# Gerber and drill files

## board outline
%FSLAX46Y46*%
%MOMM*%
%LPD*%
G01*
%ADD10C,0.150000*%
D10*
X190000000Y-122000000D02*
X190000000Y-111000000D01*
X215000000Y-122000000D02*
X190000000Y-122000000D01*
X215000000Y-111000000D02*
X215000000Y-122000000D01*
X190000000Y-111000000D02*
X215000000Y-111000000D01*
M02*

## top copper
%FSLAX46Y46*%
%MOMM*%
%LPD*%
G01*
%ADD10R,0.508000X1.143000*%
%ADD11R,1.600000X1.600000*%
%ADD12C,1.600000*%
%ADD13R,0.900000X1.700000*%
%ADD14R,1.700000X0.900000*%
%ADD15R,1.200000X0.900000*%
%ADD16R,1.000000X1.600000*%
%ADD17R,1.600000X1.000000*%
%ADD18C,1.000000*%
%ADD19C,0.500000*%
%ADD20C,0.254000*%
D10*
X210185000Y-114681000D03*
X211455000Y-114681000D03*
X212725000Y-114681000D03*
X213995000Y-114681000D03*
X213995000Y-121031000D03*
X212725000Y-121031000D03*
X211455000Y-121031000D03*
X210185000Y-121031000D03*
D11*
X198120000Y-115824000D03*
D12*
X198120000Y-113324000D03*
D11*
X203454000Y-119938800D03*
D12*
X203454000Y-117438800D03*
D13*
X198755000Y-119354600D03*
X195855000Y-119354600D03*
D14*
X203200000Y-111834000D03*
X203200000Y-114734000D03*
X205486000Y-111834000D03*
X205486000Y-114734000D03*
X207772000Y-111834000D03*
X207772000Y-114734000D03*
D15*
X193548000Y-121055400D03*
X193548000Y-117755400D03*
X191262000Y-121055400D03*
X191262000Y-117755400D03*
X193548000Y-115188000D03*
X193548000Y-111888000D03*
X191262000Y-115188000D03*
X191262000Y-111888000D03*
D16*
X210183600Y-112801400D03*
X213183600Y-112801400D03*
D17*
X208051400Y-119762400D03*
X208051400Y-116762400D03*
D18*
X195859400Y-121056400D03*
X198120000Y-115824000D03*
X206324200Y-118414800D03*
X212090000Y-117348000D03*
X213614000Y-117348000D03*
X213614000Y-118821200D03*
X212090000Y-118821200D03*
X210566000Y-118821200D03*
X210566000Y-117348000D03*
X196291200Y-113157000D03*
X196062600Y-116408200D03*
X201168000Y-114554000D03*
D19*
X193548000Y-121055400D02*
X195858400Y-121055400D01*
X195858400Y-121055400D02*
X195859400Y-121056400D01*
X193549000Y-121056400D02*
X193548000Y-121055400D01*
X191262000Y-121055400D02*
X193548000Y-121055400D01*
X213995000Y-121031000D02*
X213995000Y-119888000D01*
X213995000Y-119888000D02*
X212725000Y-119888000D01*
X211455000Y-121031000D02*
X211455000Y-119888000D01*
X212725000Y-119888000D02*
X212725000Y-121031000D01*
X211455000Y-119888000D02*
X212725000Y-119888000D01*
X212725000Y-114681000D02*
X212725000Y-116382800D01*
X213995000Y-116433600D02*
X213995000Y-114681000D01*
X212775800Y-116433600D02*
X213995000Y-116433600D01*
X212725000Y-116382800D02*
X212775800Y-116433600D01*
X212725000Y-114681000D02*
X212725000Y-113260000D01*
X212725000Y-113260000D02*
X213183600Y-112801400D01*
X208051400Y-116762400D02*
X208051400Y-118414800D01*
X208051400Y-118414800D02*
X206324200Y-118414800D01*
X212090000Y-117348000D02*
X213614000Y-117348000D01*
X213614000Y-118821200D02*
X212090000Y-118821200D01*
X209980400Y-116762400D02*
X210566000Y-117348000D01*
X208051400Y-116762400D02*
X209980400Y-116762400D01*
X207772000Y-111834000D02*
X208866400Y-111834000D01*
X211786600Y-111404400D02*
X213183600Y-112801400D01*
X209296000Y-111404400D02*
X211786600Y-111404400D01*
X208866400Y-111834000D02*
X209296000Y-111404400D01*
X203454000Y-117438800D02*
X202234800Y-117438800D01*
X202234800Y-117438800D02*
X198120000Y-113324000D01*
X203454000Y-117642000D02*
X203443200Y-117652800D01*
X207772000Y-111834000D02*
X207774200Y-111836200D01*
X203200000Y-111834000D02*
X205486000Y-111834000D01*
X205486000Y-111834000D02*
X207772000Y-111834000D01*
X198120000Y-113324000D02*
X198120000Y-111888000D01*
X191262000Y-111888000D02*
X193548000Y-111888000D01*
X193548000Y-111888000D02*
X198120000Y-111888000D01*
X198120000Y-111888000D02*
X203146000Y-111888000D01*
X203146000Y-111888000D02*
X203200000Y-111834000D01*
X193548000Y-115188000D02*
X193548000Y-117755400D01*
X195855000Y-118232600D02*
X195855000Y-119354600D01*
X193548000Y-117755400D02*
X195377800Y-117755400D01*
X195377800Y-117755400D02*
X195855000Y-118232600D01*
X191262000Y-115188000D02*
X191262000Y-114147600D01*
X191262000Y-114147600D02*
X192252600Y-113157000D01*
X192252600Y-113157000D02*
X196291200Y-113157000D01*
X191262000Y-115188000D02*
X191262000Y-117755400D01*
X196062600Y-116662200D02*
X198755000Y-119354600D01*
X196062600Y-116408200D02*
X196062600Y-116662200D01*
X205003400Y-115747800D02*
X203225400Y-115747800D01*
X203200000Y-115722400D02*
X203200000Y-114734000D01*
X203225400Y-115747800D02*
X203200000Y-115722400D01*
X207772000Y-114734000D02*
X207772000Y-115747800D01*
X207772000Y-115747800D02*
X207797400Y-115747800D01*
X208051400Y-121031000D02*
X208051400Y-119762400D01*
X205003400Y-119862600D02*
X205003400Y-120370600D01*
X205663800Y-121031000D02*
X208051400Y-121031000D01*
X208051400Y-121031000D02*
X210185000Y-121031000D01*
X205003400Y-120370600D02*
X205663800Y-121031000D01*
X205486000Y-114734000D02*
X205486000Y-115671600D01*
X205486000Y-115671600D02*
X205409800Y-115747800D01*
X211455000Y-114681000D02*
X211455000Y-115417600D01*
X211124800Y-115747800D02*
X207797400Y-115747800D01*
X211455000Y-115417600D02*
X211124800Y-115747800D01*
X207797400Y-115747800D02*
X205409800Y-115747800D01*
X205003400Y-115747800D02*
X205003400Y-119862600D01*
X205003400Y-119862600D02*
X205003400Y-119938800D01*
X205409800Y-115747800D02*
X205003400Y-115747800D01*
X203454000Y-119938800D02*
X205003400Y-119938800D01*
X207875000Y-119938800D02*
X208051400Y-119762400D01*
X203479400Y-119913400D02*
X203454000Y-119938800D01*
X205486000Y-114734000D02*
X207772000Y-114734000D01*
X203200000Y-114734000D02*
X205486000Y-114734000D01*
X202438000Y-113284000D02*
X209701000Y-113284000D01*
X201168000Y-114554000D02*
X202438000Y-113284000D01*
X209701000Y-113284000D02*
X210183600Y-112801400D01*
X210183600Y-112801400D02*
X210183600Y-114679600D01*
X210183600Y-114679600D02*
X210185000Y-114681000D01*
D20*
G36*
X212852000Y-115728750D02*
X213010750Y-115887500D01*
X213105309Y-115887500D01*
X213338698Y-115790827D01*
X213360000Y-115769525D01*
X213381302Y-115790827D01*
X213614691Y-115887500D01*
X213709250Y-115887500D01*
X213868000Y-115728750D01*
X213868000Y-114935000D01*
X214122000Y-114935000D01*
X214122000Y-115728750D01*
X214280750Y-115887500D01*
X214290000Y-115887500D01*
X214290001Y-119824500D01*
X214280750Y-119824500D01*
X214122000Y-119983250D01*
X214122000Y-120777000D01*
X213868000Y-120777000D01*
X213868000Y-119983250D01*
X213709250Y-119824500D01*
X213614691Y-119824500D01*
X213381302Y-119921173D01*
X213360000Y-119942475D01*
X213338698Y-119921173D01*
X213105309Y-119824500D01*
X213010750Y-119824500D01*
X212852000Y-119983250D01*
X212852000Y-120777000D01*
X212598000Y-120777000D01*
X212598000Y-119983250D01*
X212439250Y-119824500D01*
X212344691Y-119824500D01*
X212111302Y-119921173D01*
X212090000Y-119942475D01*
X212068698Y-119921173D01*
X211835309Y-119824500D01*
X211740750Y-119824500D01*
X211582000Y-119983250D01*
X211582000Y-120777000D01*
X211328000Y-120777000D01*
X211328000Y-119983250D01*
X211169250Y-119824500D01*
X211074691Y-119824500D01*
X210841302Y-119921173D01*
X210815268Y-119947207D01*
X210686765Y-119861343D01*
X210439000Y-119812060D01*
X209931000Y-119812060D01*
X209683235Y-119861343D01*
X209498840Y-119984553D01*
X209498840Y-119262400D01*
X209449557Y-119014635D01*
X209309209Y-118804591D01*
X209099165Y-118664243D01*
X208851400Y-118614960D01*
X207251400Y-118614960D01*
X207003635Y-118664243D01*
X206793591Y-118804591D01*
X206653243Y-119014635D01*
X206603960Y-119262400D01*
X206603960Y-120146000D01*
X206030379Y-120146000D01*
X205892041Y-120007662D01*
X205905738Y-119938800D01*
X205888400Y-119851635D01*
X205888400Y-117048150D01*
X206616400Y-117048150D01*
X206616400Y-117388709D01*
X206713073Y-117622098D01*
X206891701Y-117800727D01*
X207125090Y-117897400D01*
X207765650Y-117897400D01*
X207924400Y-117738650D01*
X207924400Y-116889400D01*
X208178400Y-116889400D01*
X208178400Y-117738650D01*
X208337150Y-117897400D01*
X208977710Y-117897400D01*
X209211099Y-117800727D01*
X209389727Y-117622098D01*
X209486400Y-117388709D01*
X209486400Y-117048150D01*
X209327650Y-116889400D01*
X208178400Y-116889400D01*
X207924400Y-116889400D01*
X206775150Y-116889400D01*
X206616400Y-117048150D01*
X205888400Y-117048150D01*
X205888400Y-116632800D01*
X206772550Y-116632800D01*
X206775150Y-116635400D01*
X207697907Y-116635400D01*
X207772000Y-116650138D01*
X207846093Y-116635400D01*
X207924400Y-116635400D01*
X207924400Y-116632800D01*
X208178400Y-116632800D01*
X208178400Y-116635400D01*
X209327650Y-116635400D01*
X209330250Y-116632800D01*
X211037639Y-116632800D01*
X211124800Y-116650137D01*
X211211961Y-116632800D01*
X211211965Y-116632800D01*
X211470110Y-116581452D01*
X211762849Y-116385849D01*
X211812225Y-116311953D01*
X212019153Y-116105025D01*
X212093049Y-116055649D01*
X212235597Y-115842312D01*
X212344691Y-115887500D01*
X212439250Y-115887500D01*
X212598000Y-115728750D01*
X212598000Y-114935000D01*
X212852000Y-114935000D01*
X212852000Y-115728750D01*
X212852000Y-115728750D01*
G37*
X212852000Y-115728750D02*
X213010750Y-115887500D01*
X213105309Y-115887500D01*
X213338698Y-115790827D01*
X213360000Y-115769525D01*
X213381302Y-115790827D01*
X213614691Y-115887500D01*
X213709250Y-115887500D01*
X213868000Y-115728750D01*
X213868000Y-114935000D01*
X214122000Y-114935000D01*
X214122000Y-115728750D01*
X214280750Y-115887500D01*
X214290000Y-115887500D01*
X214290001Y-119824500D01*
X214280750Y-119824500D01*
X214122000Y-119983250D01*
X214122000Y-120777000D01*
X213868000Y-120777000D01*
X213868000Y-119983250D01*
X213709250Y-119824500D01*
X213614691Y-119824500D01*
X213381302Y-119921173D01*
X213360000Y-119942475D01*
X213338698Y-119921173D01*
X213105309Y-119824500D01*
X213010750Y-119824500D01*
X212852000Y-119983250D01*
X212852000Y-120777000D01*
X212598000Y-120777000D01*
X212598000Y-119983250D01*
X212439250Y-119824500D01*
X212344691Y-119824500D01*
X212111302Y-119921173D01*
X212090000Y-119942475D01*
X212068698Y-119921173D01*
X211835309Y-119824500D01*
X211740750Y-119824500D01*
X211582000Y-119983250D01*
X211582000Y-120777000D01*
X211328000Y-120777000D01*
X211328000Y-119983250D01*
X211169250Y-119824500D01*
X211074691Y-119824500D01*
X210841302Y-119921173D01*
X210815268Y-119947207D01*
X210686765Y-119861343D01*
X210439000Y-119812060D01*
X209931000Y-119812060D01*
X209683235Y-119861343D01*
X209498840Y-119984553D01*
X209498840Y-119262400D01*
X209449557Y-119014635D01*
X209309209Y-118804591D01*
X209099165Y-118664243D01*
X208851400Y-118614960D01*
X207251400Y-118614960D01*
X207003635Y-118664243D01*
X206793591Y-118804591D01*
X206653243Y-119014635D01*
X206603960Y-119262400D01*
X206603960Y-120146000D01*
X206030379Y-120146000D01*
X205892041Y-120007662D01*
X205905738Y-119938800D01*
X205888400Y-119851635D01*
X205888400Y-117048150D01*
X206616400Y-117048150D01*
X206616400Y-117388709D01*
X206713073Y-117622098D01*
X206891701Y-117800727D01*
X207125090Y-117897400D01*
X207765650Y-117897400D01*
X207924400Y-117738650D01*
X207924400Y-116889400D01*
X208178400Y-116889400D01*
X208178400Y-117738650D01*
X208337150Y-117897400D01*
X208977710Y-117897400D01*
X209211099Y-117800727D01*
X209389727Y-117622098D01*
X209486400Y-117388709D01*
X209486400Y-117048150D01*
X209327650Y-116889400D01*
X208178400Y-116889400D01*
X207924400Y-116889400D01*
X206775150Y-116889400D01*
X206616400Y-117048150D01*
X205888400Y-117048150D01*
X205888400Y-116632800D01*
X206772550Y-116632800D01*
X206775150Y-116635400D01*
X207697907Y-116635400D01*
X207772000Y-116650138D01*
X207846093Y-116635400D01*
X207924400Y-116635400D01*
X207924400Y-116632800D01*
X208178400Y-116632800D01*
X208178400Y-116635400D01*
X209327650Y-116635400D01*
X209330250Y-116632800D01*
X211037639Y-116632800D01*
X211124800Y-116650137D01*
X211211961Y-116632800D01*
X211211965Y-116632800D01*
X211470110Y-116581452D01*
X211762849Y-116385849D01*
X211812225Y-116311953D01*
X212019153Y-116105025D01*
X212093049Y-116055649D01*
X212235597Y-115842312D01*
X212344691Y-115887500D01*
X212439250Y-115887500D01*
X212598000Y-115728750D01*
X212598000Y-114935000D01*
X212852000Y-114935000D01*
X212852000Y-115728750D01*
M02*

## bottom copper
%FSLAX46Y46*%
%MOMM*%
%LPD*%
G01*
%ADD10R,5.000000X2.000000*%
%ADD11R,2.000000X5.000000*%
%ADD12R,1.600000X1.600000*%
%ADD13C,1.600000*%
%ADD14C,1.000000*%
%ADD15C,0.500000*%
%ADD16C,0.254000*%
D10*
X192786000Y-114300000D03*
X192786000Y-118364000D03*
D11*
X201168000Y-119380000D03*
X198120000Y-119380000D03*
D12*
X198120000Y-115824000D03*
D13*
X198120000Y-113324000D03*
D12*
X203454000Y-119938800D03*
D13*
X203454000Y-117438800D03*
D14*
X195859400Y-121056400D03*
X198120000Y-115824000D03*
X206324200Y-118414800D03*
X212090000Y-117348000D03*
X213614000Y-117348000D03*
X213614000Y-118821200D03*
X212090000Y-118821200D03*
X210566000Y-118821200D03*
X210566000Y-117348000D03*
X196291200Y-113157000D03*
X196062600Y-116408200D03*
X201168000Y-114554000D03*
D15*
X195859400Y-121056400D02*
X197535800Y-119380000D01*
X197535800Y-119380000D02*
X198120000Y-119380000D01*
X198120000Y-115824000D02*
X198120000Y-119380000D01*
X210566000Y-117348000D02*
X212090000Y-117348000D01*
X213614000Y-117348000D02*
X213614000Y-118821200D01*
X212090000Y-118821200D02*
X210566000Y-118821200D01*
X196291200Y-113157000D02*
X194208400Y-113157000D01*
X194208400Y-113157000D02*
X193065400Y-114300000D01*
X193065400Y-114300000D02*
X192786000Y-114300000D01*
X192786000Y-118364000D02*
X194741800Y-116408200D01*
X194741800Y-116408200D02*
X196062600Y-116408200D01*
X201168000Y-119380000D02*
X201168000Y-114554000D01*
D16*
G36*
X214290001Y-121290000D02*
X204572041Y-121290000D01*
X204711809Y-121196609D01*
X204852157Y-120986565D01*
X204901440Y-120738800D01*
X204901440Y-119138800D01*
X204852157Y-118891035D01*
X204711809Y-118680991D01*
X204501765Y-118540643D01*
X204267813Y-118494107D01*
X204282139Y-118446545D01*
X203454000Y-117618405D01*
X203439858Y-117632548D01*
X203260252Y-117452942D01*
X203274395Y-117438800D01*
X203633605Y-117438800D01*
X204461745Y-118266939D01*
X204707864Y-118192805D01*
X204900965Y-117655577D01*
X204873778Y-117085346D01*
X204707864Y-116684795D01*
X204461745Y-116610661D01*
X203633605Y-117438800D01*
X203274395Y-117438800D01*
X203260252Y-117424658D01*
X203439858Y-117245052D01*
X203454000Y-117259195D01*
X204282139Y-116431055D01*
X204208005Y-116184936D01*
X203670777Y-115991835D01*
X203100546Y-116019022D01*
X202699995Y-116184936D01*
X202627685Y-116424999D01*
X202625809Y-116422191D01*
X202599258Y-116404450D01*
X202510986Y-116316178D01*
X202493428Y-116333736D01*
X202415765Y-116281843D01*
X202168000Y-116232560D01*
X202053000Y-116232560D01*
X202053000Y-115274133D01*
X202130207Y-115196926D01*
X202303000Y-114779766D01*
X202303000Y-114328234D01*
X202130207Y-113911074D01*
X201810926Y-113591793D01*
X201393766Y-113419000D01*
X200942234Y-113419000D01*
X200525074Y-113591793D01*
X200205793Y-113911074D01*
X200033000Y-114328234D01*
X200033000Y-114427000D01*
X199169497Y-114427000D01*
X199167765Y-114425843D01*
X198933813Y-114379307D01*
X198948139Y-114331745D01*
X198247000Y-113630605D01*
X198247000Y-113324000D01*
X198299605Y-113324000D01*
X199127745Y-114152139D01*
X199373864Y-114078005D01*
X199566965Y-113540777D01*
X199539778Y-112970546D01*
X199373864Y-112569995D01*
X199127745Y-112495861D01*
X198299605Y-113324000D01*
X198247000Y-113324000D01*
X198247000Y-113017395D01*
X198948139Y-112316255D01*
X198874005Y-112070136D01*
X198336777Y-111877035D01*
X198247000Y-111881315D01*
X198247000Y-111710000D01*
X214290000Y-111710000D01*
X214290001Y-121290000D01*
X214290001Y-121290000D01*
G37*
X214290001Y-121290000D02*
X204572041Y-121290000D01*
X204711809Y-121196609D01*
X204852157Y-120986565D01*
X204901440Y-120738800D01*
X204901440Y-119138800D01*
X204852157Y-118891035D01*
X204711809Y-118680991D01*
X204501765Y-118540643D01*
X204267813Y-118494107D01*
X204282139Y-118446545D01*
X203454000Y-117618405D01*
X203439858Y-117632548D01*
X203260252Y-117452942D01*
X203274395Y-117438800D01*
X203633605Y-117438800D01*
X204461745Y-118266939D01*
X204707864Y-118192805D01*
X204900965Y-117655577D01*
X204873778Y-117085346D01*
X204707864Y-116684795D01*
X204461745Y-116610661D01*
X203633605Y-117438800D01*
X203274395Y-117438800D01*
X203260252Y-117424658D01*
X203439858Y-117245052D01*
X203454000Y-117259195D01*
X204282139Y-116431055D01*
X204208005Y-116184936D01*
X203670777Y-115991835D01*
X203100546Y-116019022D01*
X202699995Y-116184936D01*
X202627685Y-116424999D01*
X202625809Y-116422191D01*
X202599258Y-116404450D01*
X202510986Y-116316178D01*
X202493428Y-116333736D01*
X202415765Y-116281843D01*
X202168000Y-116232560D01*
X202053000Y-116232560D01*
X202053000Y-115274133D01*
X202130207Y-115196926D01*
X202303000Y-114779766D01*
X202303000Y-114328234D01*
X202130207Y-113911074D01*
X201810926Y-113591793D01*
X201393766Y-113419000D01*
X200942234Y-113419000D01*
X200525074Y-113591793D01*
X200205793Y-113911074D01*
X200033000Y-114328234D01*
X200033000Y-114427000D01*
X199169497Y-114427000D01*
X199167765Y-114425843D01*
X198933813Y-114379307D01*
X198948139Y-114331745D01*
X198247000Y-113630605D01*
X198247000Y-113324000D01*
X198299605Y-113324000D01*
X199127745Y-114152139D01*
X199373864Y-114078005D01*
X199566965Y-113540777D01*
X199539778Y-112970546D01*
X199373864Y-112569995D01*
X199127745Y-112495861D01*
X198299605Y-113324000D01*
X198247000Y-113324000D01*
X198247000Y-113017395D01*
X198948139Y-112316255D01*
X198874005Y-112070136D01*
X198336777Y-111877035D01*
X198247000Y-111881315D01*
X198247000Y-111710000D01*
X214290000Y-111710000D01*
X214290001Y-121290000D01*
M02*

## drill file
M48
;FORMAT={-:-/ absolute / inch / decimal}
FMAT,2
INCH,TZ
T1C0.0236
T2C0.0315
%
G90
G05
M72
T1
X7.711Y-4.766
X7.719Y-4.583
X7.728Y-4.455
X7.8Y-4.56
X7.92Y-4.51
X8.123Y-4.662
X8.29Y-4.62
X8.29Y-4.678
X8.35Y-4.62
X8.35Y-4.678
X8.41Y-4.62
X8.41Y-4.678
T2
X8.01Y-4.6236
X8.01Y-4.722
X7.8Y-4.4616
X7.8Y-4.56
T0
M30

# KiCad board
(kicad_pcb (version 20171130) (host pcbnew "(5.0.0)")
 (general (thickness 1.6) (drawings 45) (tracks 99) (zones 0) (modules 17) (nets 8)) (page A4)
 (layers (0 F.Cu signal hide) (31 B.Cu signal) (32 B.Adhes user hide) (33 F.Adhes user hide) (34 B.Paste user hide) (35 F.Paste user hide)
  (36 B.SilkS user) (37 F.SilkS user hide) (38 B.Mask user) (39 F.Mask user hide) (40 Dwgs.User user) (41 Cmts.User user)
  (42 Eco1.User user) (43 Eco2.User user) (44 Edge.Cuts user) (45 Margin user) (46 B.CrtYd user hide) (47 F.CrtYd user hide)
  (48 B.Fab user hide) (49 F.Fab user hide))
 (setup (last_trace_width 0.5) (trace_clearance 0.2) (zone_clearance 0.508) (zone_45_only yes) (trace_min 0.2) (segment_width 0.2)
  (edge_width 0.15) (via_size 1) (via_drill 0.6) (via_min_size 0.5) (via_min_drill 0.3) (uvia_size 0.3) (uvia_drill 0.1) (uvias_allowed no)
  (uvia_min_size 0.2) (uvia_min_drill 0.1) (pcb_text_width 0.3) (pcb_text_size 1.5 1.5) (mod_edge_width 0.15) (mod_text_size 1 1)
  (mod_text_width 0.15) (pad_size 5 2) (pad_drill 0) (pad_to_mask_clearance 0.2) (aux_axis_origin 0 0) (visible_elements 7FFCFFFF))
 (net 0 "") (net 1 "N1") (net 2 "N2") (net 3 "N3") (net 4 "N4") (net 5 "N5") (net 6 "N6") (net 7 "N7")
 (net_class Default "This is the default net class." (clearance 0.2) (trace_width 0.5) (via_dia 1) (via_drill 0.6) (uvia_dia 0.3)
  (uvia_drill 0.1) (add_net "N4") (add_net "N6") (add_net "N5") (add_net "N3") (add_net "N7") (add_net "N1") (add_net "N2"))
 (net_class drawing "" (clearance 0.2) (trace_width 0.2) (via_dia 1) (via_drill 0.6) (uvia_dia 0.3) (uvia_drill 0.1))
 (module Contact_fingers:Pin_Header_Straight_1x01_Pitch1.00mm (layer F.Cu) (at 192.786 114.3 180)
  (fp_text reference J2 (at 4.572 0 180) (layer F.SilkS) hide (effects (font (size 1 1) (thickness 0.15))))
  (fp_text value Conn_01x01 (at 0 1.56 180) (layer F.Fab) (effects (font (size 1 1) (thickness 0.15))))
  (pad 1 smd rect (at 0 0 180) (size 5 2) (layers B.Cu) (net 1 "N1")))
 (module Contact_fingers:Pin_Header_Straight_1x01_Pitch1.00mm (layer F.Cu) (at 192.786 118.364 180)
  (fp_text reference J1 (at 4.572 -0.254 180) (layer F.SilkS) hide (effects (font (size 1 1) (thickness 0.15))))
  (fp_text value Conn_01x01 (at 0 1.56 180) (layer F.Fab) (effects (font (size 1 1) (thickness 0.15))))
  (pad 1 smd rect (at 0 0 180) (size 5 2) (layers B.Cu) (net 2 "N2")))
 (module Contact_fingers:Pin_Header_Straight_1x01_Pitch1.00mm (layer F.Cu) (at 201.168 119.38 270)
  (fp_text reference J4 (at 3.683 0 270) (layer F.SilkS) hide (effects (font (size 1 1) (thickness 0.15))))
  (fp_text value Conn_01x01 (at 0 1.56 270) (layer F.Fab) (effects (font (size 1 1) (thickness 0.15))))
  (pad 1 smd rect (at 0 0 270) (size 5 2) (layers B.Cu) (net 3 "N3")))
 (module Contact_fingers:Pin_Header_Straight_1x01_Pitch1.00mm (layer F.Cu) (at 198.12 119.38 270)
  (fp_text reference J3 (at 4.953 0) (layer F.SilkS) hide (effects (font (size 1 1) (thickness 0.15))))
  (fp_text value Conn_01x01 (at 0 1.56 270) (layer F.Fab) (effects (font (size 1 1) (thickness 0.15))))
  (pad 1 smd rect (at 0 0 270) (size 5 2) (layers B.Cu) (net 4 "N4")))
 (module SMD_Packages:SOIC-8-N (layer F.Cu) (at 212.09 117.856)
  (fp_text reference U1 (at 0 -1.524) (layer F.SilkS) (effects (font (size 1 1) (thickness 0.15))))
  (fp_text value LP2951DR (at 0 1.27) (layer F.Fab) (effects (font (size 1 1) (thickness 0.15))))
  (pad 8 smd rect (at -1.905 -3.175) (size 0.508 1.143) (layers F.Cu F.Paste F.Mask) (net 3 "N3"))
  (pad 7 smd rect (at -0.635 -3.175) (size 0.508 1.143) (layers F.Cu F.Paste F.Mask) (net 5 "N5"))
  (pad 6 smd rect (at 0.635 -3.175) (size 0.508 1.143) (layers F.Cu F.Paste F.Mask) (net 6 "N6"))
  (pad 5 smd rect (at 1.905 -3.175) (size 0.508 1.143) (layers F.Cu F.Paste F.Mask) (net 6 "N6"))
  (pad 4 smd rect (at 1.905 3.175) (size 0.508 1.143) (layers F.Cu F.Paste F.Mask) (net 6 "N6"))
  (pad 3 smd rect (at 0.635 3.175) (size 0.508 1.143) (layers F.Cu F.Paste F.Mask) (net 6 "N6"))
  (pad 2 smd rect (at -0.635 3.175) (size 0.508 1.143) (layers F.Cu F.Paste F.Mask) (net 6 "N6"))
  (pad 1 smd rect (at -1.905 3.175) (size 0.508 1.143) (layers F.Cu F.Paste F.Mask) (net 5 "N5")))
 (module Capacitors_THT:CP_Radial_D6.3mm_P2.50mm (layer F.Cu) (at 198.12 115.824 90)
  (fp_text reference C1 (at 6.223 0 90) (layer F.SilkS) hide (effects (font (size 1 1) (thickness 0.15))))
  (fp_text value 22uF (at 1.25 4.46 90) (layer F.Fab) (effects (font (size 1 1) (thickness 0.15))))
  (pad 1 thru_hole rect (at 0 0 90) (size 1.6 1.6) (drill 0.8) (layers *.Cu *.Mask) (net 4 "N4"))
  (pad 2 thru_hole circle (at 2.5 0 90) (size 1.6 1.6) (drill 0.8) (layers *.Cu *.Mask) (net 6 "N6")))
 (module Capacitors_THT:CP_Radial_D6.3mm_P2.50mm (layer F.Cu) (at 203.454 119.9388 90)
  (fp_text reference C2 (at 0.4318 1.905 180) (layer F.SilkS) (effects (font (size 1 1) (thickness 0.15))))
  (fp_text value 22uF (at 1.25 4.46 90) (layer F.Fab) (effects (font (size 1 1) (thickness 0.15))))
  (pad 1 thru_hole rect (at 0 0 90) (size 1.6 1.6) (drill 0.8) (layers *.Cu *.Mask) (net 5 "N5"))
  (pad 2 thru_hole circle (at 2.5 0 90) (size 1.6 1.6) (drill 0.8) (layers *.Cu *.Mask) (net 6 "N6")))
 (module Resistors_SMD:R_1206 (layer F.Cu) (at 197.305 119.3546 180)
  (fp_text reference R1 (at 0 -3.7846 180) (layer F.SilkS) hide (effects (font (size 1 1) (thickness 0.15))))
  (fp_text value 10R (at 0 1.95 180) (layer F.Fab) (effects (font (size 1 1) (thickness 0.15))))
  (pad 1 smd rect (at -1.45 0 180) (size 0.9 1.7) (layers F.Cu F.Paste F.Mask) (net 2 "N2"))
  (pad 2 smd rect (at 1.45 0 180) (size 0.9 1.7) (layers F.Cu F.Paste F.Mask) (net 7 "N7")))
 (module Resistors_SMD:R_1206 (layer F.Cu) (at 203.2 113.284 270)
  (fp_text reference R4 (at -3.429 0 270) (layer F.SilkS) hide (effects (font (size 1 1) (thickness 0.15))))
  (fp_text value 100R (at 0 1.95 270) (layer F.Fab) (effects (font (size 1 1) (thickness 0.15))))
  (pad 1 smd rect (at -1.45 0 270) (size 0.9 1.7) (layers F.Cu F.Paste F.Mask) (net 6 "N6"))
  (pad 2 smd rect (at 1.45 0 270) (size 0.9 1.7) (layers F.Cu F.Paste F.Mask) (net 5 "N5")))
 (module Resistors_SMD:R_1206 (layer F.Cu) (at 205.486 113.284 270)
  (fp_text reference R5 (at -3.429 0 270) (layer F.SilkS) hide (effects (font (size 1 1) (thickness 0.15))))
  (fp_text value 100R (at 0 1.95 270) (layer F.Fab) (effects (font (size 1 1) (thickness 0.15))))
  (pad 1 smd rect (at -1.45 0 270) (size 0.9 1.7) (layers F.Cu F.Paste F.Mask) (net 6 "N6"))
  (pad 2 smd rect (at 1.45 0 270) (size 0.9 1.7) (layers F.Cu F.Paste F.Mask) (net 5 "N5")))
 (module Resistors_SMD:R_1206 (layer F.Cu) (at 207.772 113.284 270)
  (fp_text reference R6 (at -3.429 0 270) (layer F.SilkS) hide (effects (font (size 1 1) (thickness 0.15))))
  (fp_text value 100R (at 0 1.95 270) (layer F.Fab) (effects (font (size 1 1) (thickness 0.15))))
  (pad 1 smd rect (at -1.45 0 270) (size 0.9 1.7) (layers F.Cu F.Paste F.Mask) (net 6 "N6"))
  (pad 2 smd rect (at 1.45 0 270) (size 0.9 1.7) (layers F.Cu F.Paste F.Mask) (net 5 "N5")))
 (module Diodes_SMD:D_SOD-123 (layer F.Cu) (at 193.548 119.4054 90)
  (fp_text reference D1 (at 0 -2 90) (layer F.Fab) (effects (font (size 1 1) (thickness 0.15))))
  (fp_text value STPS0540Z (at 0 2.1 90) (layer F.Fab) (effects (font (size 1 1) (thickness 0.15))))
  (pad 1 smd rect (at -1.65 0 90) (size 0.9 1.2) (layers F.Cu F.Paste F.Mask) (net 4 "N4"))
  (pad 2 smd rect (at 1.65 0 90) (size 0.9 1.2) (layers F.Cu F.Paste F.Mask) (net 7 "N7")))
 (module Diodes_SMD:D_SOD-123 (layer F.Cu) (at 191.262 119.4054 90)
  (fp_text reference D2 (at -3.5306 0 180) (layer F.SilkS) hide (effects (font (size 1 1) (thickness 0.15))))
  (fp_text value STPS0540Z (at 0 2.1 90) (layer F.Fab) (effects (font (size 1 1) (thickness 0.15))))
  (pad 1 smd rect (at -1.65 0 90) (size 0.9 1.2) (layers F.Cu F.Paste F.Mask) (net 4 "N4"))
  (pad 2 smd rect (at 1.65 0 90) (size 0.9 1.2) (layers F.Cu F.Paste F.Mask) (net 1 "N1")))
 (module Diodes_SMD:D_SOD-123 (layer F.Cu) (at 193.548 113.538 90)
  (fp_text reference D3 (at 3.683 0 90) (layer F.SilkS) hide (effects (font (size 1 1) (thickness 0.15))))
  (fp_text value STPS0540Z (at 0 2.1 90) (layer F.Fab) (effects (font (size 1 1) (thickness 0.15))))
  (pad 1 smd rect (at -1.65 0 90) (size 0.9 1.2) (layers F.Cu F.Paste F.Mask) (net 7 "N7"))
  (pad 2 smd rect (at 1.65 0 90) (size 0.9 1.2) (layers F.Cu F.Paste F.Mask) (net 6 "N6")))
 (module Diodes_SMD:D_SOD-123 (layer F.Cu) (at 191.262 113.538 90)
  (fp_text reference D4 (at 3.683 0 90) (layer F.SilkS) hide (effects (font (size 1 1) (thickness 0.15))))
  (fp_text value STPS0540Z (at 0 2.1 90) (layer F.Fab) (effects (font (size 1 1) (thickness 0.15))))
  (pad 1 smd rect (at -1.65 0 90) (size 0.9 1.2) (layers F.Cu F.Paste F.Mask) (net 1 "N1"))
  (pad 2 smd rect (at 1.65 0 90) (size 0.9 1.2) (layers F.Cu F.Paste F.Mask) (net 6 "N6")))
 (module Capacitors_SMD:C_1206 (layer F.Cu) (at 211.6836 112.8014)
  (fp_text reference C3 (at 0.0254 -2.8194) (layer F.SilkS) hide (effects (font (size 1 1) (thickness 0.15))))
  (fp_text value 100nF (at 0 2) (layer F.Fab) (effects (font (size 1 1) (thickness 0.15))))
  (pad 1 smd rect (at -1.5 0) (size 1 1.6) (layers F.Cu F.Paste F.Mask) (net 3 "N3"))
  (pad 2 smd rect (at 1.5 0) (size 1 1.6) (layers F.Cu F.Paste F.Mask) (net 6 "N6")))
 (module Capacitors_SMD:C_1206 (layer F.Cu) (at 208.0514 118.2624 90)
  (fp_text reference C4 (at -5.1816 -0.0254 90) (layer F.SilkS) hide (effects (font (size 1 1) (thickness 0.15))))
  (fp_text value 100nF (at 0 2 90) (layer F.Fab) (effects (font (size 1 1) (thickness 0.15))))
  (pad 1 smd rect (at -1.5 0 90) (size 1 1.6) (layers F.Cu F.Paste F.Mask) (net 5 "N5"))
  (pad 2 smd rect (at 1.5 0 90) (size 1 1.6) (layers F.Cu F.Paste F.Mask) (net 6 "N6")))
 (gr_line (start 190 122) (end 190 111) (angle 90) (layer Edge.Cuts) (width 0.15))
 (gr_line (start 215 122) (end 190 122) (angle 90) (layer Edge.Cuts) (width 0.15))
 (gr_line (start 215 111) (end 215 122) (angle 90) (layer Edge.Cuts) (width 0.15))
 (gr_line (start 190 111) (end 215 111) (angle 90) (layer Edge.Cuts) (width 0.15))
 (segment (start 193.548 121.0554) (end 195.8584 121.0554) (width 0.5) (layer F.Cu) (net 4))
 (segment (start 195.8584 121.0554) (end 195.8594 121.0564) (width 0.5) (layer F.Cu) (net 4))
 (via (at 195.8594 121.0564) (size 1) (drill 0.6) (layers F.Cu B.Cu) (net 4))
 (segment (start 195.8594 121.0564) (end 197.5358 119.38) (width 0.5) (layer B.Cu) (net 4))
 (segment (start 197.5358 119.38) (end 198.12 119.38) (width 0.5) (layer B.Cu) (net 4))
 (segment (start 193.549 121.0564) (end 193.548 121.0554) (width 0.5) (layer F.Cu) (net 4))
 (segment (start 191.262 121.0554) (end 193.548 121.0554) (width 0.5) (layer F.Cu) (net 4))
 (via (at 198.12 115.824) (size 1) (drill 0.6) (layers F.Cu B.Cu) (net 4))
 (segment (start 198.12 115.824) (end 198.12 119.38) (width 0.5) (layer B.Cu) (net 4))
 (segment (start 213.995 121.031) (end 213.995 119.888) (width 0.5) (layer F.Cu) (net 6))
 (segment (start 213.995 119.888) (end 212.725 119.888) (width 0.5) (layer F.Cu) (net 6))
 (segment (start 211.455 121.031) (end 211.455 119.888) (width 0.5) (layer F.Cu) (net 6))
 (segment (start 212.725 119.888) (end 212.725 121.031) (width 0.5) (layer F.Cu) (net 6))
 (segment (start 211.455 119.888) (end 212.725 119.888) (width 0.5) (layer F.Cu) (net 6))
 (segment (start 212.725 114.681) (end 212.725 116.3828) (width 0.5) (layer F.Cu) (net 6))
 (segment (start 213.995 116.4336) (end 213.995 114.681) (width 0.5) (layer F.Cu) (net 6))
 (segment (start 212.7758 116.4336) (end 213.995 116.4336) (width 0.5) (layer F.Cu) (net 6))
 (segment (start 212.725 116.3828) (end 212.7758 116.4336) (width 0.5) (layer F.Cu) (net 6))
 (segment (start 212.725 114.681) (end 212.725 113.26) (width 0.5) (layer F.Cu) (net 6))
 (segment (start 212.725 113.26) (end 213.1836 112.8014) (width 0.5) (layer F.Cu) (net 6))
 (segment (start 208.0514 116.7624) (end 208.0514 118.4148) (width 0.5) (layer F.Cu) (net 6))
 (segment (start 208.0514 118.4148) (end 206.3242 118.4148) (width 0.5) (layer F.Cu) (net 6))
 (via (at 206.3242 118.4148) (size 1) (drill 0.6) (layers F.Cu B.Cu) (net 6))
 (segment (start 210.566 117.348) (end 212.09 117.348) (width 0.5) (layer B.Cu) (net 6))
 (via (at 212.09 117.348) (size 1) (drill 0.6) (layers F.Cu B.Cu) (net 6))
 (segment (start 212.09 117.348) (end 213.614 117.348) (width 0.5) (layer F.Cu) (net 6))
 (via (at 213.614 117.348) (size 1) (drill 0.6) (layers F.Cu B.Cu) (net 6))
 (segment (start 213.614 117.348) (end 213.614 118.8212) (width 0.5) (layer B.Cu) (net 6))
 (via (at 213.614 118.8212) (size 1) (drill 0.6) (layers F.Cu B.Cu) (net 6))
 (segment (start 213.614 118.8212) (end 212.09 118.8212) (width 0.5) (layer F.Cu) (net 6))
 (via (at 212.09 118.8212) (size 1) (drill 0.6) (layers F.Cu B.Cu) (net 6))
 (segment (start 212.09 118.8212) (end 210.566 118.8212) (width 0.5) (layer B.Cu) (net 6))
 (via (at 210.566 118.8212) (size 1) (drill 0.6) (layers F.Cu B.Cu) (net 6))
 (via (at 210.566 117.348) (size 1) (drill 0.6) (layers F.Cu B.Cu) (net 6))
 (segment (start 209.9804 116.7624) (end 210.566 117.348) (width 0.5) (layer F.Cu) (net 6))
 (segment (start 208.0514 116.7624) (end 209.9804 116.7624) (width 0.5) (layer F.Cu) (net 6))
 (segment (start 207.772 111.834) (end 208.8664 111.834) (width 0.5) (layer F.Cu) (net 6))
 (segment (start 211.7866 111.4044) (end 213.1836 112.8014) (width 0.5) (layer F.Cu) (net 6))
 (segment (start 209.296 111.4044) (end 211.7866 111.4044) (width 0.5) (layer F.Cu) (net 6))
 (segment (start 208.8664 111.834) (end 209.296 111.4044) (width 0.5) (layer F.Cu) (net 6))
 (segment (start 203.454 117.4388) (end 202.2348 117.4388) (width 0.5) (layer F.Cu) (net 6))
 (segment (start 202.2348 117.4388) (end 198.12 113.324) (width 0.5) (layer F.Cu) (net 6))
 (segment (start 203.454 117.642) (end 203.4432 117.6528) (width 0.5) (layer F.Cu) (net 6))
 (segment (start 207.772 111.834) (end 207.7742 111.8362) (width 0.5) (layer F.Cu) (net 6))
 (segment (start 203.2 111.834) (end 205.486 111.834) (width 0.5) (layer F.Cu) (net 6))
 (segment (start 205.486 111.834) (end 207.772 111.834) (width 0.5) (layer F.Cu) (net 6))
 (segment (start 198.12 113.324) (end 198.12 111.888) (width 0.5) (layer F.Cu) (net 6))
 (segment (start 191.262 111.888) (end 193.548 111.888) (width 0.5) (layer F.Cu) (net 6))
 (segment (start 193.548 111.888) (end 198.12 111.888) (width 0.5) (layer F.Cu) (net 6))
 (segment (start 198.12 111.888) (end 203.146 111.888) (width 0.5) (layer F.Cu) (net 6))
 (segment (start 203.146 111.888) (end 203.2 111.834) (width 0.5) (layer F.Cu) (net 6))
 (segment (start 193.548 115.188) (end 193.548 117.7554) (width 0.5) (layer F.Cu) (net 7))
 (segment (start 195.855 118.2326) (end 195.855 119.3546) (width 0.5) (layer F.Cu) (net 7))
 (segment (start 193.548 117.7554) (end 195.3778 117.7554) (width 0.5) (layer F.Cu) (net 7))
 (segment (start 195.3778 117.7554) (end 195.855 118.2326) (width 0.5) (layer F.Cu) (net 7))
 (segment (start 191.262 115.188) (end 191.262 114.1476) (width 0.5) (layer F.Cu) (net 1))
 (segment (start 191.262 114.1476) (end 192.2526 113.157) (width 0.5) (layer F.Cu) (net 1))
 (segment (start 192.2526 113.157) (end 196.2912 113.157) (width 0.5) (layer F.Cu) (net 1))
 (via (at 196.2912 113.157) (size 1) (drill 0.6) (layers F.Cu B.Cu) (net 1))
 (segment (start 196.2912 113.157) (end 194.2084 113.157) (width 0.5) (layer B.Cu) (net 1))
 (segment (start 194.2084 113.157) (end 193.0654 114.3) (width 0.5) (layer B.Cu) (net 1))
 (segment (start 193.0654 114.3) (end 192.786 114.3) (width 0.5) (layer B.Cu) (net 1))
 (segment (start 191.262 115.188) (end 191.262 117.7554) (width 0.5) (layer F.Cu) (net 1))
 (segment (start 192.786 118.364) (end 194.7418 116.4082) (width 0.5) (layer B.Cu) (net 2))
 (via (at 196.0626 116.4082) (size 1) (drill 0.6) (layers F.Cu B.Cu) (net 2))
 (segment (start 194.7418 116.4082) (end 196.0626 116.4082) (width 0.5) (layer B.Cu) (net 2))
 (segment (start 196.0626 116.6622) (end 198.755 119.3546) (width 0.5) (layer F.Cu) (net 2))
 (segment (start 196.0626 116.4082) (end 196.0626 116.6622) (width 0.5) (layer F.Cu) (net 2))
 (segment (start 205.0034 115.7478) (end 203.2254 115.7478) (width 0.5) (layer F.Cu) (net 5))
 (segment (start 203.2 115.7224) (end 203.2 114.734) (width 0.5) (layer F.Cu) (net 5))
 (segment (start 203.2254 115.7478) (end 203.2 115.7224) (width 0.5) (layer F.Cu) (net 5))
 (segment (start 207.772 114.734) (end 207.772 115.7478) (width 0.5) (layer F.Cu) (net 5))
 (segment (start 207.772 115.7478) (end 207.7974 115.7478) (width 0.5) (layer F.Cu) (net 5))
 (segment (start 208.0514 121.031) (end 208.0514 119.7624) (width 0.5) (layer F.Cu) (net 5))
 (segment (start 205.0034 119.8626) (end 205.0034 120.3706) (width 0.5) (layer F.Cu) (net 5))
 (segment (start 205.6638 121.031) (end 208.0514 121.031) (width 0.5) (layer F.Cu) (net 5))
 (segment (start 208.0514 121.031) (end 210.185 121.031) (width 0.5) (layer F.Cu) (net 5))
 (segment (start 205.0034 120.3706) (end 205.6638 121.031) (width 0.5) (layer F.Cu) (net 5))
 (segment (start 205.486 114.734) (end 205.486 115.6716) (width 0.5) (layer F.Cu) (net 5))
 (segment (start 205.486 115.6716) (end 205.4098 115.7478) (width 0.5) (layer F.Cu) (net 5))
 (segment (start 211.455 114.681) (end 211.455 115.4176) (width 0.5) (layer F.Cu) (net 5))
 (segment (start 211.1248 115.7478) (end 207.7974 115.7478) (width 0.5) (layer F.Cu) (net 5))
 (segment (start 211.455 115.4176) (end 211.1248 115.7478) (width 0.5) (layer F.Cu) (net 5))
 (segment (start 207.7974 115.7478) (end 205.4098 115.7478) (width 0.5) (layer F.Cu) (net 5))
 (segment (start 205.0034 115.7478) (end 205.0034 119.8626) (width 0.5) (layer F.Cu) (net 5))
 (segment (start 205.0034 119.8626) (end 205.0034 119.9388) (width 0.5) (layer F.Cu) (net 5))
 (segment (start 205.4098 115.7478) (end 205.0034 115.7478) (width 0.5) (layer F.Cu) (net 5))
 (segment (start 203.454 119.9388) (end 205.0034 119.9388) (width 0.5) (layer F.Cu) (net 5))
 (segment (start 207.875 119.9388) (end 208.0514 119.7624) (width 0.5) (layer F.Cu) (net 5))
 (segment (start 203.4794 119.9134) (end 203.454 119.9388) (width 0.5) (layer F.Cu) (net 5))
 (segment (start 205.486 114.734) (end 207.772 114.734) (width 0.5) (layer F.Cu) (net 5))
 (segment (start 203.2 114.734) (end 205.486 114.734) (width 0.5) (layer F.Cu) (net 5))
 (segment (start 201.168 119.38) (end 201.168 114.554) (width 0.5) (layer B.Cu) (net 3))
 (segment (start 202.438 113.284) (end 209.701 113.284) (width 0.5) (layer F.Cu) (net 3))
 (segment (start 201.168 114.554) (end 202.438 113.284) (width 0.5) (layer F.Cu) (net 3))
 (via (at 201.168 114.554) (size 1) (drill 0.6) (layers F.Cu B.Cu) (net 3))
 (segment (start 209.701 113.284) (end 210.1836 112.8014) (width 0.5) (layer F.Cu) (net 3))
 (segment (start 210.1836 112.8014) (end 210.1836 114.6796) (width 0.5) (layer F.Cu) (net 3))
 (segment (start 210.1836 114.6796) (end 210.185 114.681) (width 0.5) (layer F.Cu) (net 3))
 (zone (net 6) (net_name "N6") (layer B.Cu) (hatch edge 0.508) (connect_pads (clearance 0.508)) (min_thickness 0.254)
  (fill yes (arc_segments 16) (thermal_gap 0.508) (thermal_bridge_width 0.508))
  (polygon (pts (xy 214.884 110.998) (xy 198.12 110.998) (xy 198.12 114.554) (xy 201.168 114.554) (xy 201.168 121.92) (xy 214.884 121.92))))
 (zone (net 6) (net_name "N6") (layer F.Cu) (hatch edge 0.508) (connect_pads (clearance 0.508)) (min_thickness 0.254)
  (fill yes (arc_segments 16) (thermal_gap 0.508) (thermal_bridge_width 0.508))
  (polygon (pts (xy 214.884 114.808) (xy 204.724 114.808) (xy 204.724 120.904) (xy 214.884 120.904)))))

